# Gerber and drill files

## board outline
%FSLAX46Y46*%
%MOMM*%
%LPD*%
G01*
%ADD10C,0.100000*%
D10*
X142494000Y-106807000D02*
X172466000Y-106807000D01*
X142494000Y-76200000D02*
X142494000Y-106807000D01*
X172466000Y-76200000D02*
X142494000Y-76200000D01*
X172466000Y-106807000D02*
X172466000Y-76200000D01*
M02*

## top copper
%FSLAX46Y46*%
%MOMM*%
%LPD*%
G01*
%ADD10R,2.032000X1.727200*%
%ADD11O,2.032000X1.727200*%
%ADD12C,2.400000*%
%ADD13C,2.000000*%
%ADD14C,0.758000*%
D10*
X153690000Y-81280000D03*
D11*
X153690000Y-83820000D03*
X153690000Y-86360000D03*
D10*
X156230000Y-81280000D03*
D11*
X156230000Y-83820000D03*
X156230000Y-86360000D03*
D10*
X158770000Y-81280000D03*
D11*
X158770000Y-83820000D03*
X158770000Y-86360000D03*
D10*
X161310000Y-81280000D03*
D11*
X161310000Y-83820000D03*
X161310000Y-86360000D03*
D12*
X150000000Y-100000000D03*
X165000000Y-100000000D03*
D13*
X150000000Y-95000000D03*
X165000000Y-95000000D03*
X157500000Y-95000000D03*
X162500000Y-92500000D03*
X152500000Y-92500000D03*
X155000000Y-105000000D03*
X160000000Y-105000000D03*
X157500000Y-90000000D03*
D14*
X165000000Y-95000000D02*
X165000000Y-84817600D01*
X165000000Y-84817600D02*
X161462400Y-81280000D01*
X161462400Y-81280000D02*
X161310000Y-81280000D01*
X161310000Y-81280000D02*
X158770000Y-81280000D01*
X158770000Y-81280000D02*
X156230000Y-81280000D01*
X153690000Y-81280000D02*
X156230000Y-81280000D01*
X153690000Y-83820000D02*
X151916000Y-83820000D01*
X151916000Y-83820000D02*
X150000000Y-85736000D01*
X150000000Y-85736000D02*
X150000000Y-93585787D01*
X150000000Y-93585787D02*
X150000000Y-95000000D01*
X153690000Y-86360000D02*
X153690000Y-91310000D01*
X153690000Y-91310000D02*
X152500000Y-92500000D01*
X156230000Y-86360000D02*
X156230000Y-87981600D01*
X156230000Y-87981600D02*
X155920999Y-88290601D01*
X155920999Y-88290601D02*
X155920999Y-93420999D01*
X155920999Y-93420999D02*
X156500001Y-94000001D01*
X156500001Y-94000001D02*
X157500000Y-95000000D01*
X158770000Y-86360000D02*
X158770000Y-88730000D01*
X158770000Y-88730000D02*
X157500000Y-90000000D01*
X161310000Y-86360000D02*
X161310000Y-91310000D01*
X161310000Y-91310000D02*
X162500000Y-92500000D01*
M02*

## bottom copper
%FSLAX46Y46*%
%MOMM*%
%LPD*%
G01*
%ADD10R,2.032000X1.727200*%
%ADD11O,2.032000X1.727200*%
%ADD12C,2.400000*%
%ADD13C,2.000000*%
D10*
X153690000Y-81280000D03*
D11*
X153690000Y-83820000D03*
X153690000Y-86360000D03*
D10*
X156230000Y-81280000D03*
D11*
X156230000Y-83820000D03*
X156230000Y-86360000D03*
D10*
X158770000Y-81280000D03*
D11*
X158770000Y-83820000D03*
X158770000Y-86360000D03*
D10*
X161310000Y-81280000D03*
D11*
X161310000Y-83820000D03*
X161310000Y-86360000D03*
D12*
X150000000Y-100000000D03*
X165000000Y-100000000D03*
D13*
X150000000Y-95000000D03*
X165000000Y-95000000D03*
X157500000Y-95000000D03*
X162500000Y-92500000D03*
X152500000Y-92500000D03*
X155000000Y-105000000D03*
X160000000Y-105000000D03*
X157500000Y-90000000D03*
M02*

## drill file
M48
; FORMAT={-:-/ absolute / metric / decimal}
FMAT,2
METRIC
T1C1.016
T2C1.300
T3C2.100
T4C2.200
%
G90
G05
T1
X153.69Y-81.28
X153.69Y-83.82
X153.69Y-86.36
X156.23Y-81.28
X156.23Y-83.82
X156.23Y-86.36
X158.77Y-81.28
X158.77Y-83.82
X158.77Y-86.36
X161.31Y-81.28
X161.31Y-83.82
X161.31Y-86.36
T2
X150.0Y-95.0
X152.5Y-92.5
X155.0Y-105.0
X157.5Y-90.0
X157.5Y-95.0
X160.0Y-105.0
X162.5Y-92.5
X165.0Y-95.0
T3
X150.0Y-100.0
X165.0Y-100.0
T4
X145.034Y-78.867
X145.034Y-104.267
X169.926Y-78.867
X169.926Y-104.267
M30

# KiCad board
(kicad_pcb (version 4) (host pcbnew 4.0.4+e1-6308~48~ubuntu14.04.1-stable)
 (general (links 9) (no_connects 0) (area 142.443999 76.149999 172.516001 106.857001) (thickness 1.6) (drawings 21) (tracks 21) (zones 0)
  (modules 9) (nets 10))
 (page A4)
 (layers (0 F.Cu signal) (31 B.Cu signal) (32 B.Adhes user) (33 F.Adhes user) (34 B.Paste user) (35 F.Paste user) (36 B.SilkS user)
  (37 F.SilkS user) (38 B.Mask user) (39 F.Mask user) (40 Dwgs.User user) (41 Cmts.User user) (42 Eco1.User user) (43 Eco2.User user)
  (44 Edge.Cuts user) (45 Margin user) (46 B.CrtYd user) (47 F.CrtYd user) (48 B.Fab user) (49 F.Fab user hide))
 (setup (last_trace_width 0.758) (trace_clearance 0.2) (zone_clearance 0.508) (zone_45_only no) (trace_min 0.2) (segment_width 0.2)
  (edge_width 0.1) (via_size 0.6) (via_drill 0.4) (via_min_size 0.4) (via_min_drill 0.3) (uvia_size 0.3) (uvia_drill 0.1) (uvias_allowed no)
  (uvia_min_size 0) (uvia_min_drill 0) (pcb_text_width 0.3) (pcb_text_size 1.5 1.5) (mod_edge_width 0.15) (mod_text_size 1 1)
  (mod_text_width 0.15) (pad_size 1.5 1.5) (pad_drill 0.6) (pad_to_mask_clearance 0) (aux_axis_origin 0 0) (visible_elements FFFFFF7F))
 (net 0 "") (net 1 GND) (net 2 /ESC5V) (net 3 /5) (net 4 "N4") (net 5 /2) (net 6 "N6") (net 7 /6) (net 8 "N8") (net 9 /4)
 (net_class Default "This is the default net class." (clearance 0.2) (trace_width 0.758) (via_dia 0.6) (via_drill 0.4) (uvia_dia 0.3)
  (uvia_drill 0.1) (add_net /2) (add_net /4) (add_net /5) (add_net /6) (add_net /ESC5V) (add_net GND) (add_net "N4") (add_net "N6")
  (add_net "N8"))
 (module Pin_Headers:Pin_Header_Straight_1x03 (layer F.Cu) (at 153.69 81.28)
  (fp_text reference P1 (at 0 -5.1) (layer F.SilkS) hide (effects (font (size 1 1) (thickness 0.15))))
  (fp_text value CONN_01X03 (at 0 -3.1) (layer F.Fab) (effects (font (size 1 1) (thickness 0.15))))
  (pad 1 thru_hole rect (at 0 0) (size 2.032 1.7272) (drill 1.016) (layers *.Cu *.Mask F.SilkS) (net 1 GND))
  (pad 2 thru_hole oval (at 0 2.54) (size 2.032 1.7272) (drill 1.016) (layers *.Cu *.Mask F.SilkS) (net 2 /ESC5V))
  (pad 3 thru_hole oval (at 0 5.08) (size 2.032 1.7272) (drill 1.016) (layers *.Cu *.Mask F.SilkS) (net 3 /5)))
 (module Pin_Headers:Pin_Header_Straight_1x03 (layer F.Cu) (at 156.23 81.28)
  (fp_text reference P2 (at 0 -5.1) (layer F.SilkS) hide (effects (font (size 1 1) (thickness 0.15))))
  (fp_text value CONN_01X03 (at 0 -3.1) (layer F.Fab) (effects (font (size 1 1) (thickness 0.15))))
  (pad 1 thru_hole rect (at 0 0) (size 2.032 1.7272) (drill 1.016) (layers *.Cu *.Mask F.SilkS) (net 1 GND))
  (pad 2 thru_hole oval (at 0 2.54) (size 2.032 1.7272) (drill 1.016) (layers *.Cu *.Mask F.SilkS) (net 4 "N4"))
  (pad 3 thru_hole oval (at 0 5.08) (size 2.032 1.7272) (drill 1.016) (layers *.Cu *.Mask F.SilkS) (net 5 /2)))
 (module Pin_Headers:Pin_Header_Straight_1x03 (layer F.Cu) (at 158.77 81.28)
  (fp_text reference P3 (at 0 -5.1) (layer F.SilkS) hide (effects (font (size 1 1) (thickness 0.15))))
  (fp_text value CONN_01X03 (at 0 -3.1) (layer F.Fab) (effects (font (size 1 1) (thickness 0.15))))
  (pad 1 thru_hole rect (at 0 0) (size 2.032 1.7272) (drill 1.016) (layers *.Cu *.Mask F.SilkS) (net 1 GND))
  (pad 2 thru_hole oval (at 0 2.54) (size 2.032 1.7272) (drill 1.016) (layers *.Cu *.Mask F.SilkS) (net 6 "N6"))
  (pad 3 thru_hole oval (at 0 5.08) (size 2.032 1.7272) (drill 1.016) (layers *.Cu *.Mask F.SilkS) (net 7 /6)))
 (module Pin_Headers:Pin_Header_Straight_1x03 (layer F.Cu) (at 161.31 81.28)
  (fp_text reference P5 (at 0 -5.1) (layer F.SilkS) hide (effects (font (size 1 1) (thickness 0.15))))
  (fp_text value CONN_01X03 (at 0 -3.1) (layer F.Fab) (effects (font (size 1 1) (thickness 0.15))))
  (pad 1 thru_hole rect (at 0 0) (size 2.032 1.7272) (drill 1.016) (layers *.Cu *.Mask F.SilkS) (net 1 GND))
  (pad 2 thru_hole oval (at 0 2.54) (size 2.032 1.7272) (drill 1.016) (layers *.Cu *.Mask F.SilkS) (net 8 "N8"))
  (pad 3 thru_hole oval (at 0 5.08) (size 2.032 1.7272) (drill 1.016) (layers *.Cu *.Mask F.SilkS) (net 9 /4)))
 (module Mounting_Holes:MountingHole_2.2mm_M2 (layer F.Cu) (at 169.926 104.267)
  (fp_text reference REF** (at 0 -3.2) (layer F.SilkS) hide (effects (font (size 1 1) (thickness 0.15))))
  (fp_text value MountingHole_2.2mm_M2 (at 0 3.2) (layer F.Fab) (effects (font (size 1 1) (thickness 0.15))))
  (pad 1 np_thru_hole circle (at 0 0) (size 2.2 2.2) (drill 2.2) (layers *.Cu *.Mask F.SilkS)))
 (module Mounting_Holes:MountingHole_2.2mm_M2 (layer F.Cu) (at 145.034 104.267)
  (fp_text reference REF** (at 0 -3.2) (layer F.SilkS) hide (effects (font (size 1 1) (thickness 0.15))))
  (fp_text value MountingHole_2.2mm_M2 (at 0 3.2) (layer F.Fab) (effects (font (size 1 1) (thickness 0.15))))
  (pad 1 np_thru_hole circle (at 0 0) (size 2.2 2.2) (drill 2.2) (layers *.Cu *.Mask F.SilkS)))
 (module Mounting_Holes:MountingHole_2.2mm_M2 (layer F.Cu) (at 169.926 78.867)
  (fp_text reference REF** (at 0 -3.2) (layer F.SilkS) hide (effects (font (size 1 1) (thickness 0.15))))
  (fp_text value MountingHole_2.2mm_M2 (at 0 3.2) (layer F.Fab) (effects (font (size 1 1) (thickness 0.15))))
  (pad 1 np_thru_hole circle (at 0 0) (size 2.2 2.2) (drill 2.2) (layers *.Cu *.Mask F.SilkS)))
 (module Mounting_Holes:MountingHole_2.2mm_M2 (layer F.Cu) (at 145.034 78.867)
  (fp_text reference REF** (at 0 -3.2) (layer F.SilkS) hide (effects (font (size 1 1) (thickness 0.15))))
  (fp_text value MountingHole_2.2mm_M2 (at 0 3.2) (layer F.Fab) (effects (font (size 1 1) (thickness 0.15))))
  (pad 1 np_thru_hole circle (at 0 0) (size 2.2 2.2) (drill 2.2) (layers *.Cu *.Mask F.SilkS)))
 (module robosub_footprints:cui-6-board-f (layer F.Cu) (at 150 100)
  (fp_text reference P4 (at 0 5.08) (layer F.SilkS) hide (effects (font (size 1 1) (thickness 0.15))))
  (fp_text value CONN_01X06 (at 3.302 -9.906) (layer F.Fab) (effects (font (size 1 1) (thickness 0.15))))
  (pad ~ thru_hole circle (at 0 0) (size 2.4 2.4) (drill 2.1) (layers *.Cu *.Mask F.SilkS))
  (pad ~ thru_hole circle (at 15 0) (size 2.4 2.4) (drill 2.1) (layers *.Cu *.Mask F.SilkS))
  (pad 3 thru_hole circle (at 0 -5) (size 2 2) (drill 1.3) (layers *.Cu *.Mask F.SilkS) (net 2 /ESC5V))
  (pad 1 thru_hole circle (at 15 -5) (size 2 2) (drill 1.3) (layers *.Cu *.Mask F.SilkS) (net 1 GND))
  (pad 2 thru_hole circle (at 7.5 -5) (size 2 2) (drill 1.3) (layers *.Cu *.Mask F.SilkS) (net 5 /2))
  (pad 4 thru_hole circle (at 12.5 -7.5) (size 2 2) (drill 1.3) (layers *.Cu *.Mask F.SilkS) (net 9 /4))
  (pad 5 thru_hole circle (at 2.5 -7.5) (size 2 2) (drill 1.3) (layers *.Cu *.Mask F.SilkS) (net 3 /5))
  (pad ~ thru_hole circle (at 5 5) (size 2 2) (drill 1.3) (layers *.Cu *.Mask F.SilkS))
  (pad ~ thru_hole circle (at 10 5) (size 2 2) (drill 1.3) (layers *.Cu *.Mask F.SilkS))
  (pad 6 thru_hole circle (at 7.5 -10) (size 2 2) (drill 1.3) (layers *.Cu *.Mask F.SilkS) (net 7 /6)))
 (gr_line (start 142.494 106.807) (end 172.466 106.807) (layer Edge.Cuts) (width 0.1))
 (gr_line (start 142.494 76.2) (end 142.494 106.807) (layer Edge.Cuts) (width 0.1))
 (gr_line (start 172.466 76.2) (end 142.494 76.2) (layer Edge.Cuts) (width 0.1))
 (gr_line (start 172.466 106.807) (end 172.466 76.2) (layer Edge.Cuts) (width 0.1))
 (segment (start 165 95) (end 165 84.8176) (width 0.758) (layer F.Cu) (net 1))
 (segment (start 165 84.8176) (end 161.4624 81.28) (width 0.758) (layer F.Cu) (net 1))
 (segment (start 161.4624 81.28) (end 161.31 81.28) (width 0.758) (layer F.Cu) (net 1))
 (segment (start 161.31 81.28) (end 158.77 81.28) (width 0.758) (layer F.Cu) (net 1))
 (segment (start 158.77 81.28) (end 156.23 81.28) (width 0.758) (layer F.Cu) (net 1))
 (segment (start 153.69 81.28) (end 156.23 81.28) (width 0.758) (layer F.Cu) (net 1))
 (segment (start 153.69 83.82) (end 151.916 83.82) (width 0.758) (layer F.Cu) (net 2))
 (segment (start 151.916 83.82) (end 150 85.736) (width 0.758) (layer F.Cu) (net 2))
 (segment (start 150 85.736) (end 150 93.585787) (width 0.758) (layer F.Cu) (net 2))
 (segment (start 150 93.585787) (end 150 95) (width 0.758) (layer F.Cu) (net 2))
 (segment (start 153.69 86.36) (end 153.69 91.31) (width 0.758) (layer F.Cu) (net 3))
 (segment (start 153.69 91.31) (end 152.5 92.5) (width 0.758) (layer F.Cu) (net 3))
 (segment (start 156.23 86.36) (end 156.23 87.9816) (width 0.758) (layer F.Cu) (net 5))
 (segment (start 156.23 87.9816) (end 155.920999 88.290601) (width 0.758) (layer F.Cu) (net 5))
 (segment (start 155.920999 88.290601) (end 155.920999 93.420999) (width 0.758) (layer F.Cu) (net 5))
 (segment (start 155.920999 93.420999) (end 156.500001 94.000001) (width 0.758) (layer F.Cu) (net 5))
 (segment (start 156.500001 94.000001) (end 157.5 95) (width 0.758) (layer F.Cu) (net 5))
 (segment (start 158.77 86.36) (end 158.77 88.73) (width 0.758) (layer F.Cu) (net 7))
 (segment (start 158.77 88.73) (end 157.5 90) (width 0.758) (layer F.Cu) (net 7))
 (segment (start 161.31 86.36) (end 161.31 91.31) (width 0.758) (layer F.Cu) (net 9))
 (segment (start 161.31 91.31) (end 162.5 92.5) (width 0.758) (layer F.Cu) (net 9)))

